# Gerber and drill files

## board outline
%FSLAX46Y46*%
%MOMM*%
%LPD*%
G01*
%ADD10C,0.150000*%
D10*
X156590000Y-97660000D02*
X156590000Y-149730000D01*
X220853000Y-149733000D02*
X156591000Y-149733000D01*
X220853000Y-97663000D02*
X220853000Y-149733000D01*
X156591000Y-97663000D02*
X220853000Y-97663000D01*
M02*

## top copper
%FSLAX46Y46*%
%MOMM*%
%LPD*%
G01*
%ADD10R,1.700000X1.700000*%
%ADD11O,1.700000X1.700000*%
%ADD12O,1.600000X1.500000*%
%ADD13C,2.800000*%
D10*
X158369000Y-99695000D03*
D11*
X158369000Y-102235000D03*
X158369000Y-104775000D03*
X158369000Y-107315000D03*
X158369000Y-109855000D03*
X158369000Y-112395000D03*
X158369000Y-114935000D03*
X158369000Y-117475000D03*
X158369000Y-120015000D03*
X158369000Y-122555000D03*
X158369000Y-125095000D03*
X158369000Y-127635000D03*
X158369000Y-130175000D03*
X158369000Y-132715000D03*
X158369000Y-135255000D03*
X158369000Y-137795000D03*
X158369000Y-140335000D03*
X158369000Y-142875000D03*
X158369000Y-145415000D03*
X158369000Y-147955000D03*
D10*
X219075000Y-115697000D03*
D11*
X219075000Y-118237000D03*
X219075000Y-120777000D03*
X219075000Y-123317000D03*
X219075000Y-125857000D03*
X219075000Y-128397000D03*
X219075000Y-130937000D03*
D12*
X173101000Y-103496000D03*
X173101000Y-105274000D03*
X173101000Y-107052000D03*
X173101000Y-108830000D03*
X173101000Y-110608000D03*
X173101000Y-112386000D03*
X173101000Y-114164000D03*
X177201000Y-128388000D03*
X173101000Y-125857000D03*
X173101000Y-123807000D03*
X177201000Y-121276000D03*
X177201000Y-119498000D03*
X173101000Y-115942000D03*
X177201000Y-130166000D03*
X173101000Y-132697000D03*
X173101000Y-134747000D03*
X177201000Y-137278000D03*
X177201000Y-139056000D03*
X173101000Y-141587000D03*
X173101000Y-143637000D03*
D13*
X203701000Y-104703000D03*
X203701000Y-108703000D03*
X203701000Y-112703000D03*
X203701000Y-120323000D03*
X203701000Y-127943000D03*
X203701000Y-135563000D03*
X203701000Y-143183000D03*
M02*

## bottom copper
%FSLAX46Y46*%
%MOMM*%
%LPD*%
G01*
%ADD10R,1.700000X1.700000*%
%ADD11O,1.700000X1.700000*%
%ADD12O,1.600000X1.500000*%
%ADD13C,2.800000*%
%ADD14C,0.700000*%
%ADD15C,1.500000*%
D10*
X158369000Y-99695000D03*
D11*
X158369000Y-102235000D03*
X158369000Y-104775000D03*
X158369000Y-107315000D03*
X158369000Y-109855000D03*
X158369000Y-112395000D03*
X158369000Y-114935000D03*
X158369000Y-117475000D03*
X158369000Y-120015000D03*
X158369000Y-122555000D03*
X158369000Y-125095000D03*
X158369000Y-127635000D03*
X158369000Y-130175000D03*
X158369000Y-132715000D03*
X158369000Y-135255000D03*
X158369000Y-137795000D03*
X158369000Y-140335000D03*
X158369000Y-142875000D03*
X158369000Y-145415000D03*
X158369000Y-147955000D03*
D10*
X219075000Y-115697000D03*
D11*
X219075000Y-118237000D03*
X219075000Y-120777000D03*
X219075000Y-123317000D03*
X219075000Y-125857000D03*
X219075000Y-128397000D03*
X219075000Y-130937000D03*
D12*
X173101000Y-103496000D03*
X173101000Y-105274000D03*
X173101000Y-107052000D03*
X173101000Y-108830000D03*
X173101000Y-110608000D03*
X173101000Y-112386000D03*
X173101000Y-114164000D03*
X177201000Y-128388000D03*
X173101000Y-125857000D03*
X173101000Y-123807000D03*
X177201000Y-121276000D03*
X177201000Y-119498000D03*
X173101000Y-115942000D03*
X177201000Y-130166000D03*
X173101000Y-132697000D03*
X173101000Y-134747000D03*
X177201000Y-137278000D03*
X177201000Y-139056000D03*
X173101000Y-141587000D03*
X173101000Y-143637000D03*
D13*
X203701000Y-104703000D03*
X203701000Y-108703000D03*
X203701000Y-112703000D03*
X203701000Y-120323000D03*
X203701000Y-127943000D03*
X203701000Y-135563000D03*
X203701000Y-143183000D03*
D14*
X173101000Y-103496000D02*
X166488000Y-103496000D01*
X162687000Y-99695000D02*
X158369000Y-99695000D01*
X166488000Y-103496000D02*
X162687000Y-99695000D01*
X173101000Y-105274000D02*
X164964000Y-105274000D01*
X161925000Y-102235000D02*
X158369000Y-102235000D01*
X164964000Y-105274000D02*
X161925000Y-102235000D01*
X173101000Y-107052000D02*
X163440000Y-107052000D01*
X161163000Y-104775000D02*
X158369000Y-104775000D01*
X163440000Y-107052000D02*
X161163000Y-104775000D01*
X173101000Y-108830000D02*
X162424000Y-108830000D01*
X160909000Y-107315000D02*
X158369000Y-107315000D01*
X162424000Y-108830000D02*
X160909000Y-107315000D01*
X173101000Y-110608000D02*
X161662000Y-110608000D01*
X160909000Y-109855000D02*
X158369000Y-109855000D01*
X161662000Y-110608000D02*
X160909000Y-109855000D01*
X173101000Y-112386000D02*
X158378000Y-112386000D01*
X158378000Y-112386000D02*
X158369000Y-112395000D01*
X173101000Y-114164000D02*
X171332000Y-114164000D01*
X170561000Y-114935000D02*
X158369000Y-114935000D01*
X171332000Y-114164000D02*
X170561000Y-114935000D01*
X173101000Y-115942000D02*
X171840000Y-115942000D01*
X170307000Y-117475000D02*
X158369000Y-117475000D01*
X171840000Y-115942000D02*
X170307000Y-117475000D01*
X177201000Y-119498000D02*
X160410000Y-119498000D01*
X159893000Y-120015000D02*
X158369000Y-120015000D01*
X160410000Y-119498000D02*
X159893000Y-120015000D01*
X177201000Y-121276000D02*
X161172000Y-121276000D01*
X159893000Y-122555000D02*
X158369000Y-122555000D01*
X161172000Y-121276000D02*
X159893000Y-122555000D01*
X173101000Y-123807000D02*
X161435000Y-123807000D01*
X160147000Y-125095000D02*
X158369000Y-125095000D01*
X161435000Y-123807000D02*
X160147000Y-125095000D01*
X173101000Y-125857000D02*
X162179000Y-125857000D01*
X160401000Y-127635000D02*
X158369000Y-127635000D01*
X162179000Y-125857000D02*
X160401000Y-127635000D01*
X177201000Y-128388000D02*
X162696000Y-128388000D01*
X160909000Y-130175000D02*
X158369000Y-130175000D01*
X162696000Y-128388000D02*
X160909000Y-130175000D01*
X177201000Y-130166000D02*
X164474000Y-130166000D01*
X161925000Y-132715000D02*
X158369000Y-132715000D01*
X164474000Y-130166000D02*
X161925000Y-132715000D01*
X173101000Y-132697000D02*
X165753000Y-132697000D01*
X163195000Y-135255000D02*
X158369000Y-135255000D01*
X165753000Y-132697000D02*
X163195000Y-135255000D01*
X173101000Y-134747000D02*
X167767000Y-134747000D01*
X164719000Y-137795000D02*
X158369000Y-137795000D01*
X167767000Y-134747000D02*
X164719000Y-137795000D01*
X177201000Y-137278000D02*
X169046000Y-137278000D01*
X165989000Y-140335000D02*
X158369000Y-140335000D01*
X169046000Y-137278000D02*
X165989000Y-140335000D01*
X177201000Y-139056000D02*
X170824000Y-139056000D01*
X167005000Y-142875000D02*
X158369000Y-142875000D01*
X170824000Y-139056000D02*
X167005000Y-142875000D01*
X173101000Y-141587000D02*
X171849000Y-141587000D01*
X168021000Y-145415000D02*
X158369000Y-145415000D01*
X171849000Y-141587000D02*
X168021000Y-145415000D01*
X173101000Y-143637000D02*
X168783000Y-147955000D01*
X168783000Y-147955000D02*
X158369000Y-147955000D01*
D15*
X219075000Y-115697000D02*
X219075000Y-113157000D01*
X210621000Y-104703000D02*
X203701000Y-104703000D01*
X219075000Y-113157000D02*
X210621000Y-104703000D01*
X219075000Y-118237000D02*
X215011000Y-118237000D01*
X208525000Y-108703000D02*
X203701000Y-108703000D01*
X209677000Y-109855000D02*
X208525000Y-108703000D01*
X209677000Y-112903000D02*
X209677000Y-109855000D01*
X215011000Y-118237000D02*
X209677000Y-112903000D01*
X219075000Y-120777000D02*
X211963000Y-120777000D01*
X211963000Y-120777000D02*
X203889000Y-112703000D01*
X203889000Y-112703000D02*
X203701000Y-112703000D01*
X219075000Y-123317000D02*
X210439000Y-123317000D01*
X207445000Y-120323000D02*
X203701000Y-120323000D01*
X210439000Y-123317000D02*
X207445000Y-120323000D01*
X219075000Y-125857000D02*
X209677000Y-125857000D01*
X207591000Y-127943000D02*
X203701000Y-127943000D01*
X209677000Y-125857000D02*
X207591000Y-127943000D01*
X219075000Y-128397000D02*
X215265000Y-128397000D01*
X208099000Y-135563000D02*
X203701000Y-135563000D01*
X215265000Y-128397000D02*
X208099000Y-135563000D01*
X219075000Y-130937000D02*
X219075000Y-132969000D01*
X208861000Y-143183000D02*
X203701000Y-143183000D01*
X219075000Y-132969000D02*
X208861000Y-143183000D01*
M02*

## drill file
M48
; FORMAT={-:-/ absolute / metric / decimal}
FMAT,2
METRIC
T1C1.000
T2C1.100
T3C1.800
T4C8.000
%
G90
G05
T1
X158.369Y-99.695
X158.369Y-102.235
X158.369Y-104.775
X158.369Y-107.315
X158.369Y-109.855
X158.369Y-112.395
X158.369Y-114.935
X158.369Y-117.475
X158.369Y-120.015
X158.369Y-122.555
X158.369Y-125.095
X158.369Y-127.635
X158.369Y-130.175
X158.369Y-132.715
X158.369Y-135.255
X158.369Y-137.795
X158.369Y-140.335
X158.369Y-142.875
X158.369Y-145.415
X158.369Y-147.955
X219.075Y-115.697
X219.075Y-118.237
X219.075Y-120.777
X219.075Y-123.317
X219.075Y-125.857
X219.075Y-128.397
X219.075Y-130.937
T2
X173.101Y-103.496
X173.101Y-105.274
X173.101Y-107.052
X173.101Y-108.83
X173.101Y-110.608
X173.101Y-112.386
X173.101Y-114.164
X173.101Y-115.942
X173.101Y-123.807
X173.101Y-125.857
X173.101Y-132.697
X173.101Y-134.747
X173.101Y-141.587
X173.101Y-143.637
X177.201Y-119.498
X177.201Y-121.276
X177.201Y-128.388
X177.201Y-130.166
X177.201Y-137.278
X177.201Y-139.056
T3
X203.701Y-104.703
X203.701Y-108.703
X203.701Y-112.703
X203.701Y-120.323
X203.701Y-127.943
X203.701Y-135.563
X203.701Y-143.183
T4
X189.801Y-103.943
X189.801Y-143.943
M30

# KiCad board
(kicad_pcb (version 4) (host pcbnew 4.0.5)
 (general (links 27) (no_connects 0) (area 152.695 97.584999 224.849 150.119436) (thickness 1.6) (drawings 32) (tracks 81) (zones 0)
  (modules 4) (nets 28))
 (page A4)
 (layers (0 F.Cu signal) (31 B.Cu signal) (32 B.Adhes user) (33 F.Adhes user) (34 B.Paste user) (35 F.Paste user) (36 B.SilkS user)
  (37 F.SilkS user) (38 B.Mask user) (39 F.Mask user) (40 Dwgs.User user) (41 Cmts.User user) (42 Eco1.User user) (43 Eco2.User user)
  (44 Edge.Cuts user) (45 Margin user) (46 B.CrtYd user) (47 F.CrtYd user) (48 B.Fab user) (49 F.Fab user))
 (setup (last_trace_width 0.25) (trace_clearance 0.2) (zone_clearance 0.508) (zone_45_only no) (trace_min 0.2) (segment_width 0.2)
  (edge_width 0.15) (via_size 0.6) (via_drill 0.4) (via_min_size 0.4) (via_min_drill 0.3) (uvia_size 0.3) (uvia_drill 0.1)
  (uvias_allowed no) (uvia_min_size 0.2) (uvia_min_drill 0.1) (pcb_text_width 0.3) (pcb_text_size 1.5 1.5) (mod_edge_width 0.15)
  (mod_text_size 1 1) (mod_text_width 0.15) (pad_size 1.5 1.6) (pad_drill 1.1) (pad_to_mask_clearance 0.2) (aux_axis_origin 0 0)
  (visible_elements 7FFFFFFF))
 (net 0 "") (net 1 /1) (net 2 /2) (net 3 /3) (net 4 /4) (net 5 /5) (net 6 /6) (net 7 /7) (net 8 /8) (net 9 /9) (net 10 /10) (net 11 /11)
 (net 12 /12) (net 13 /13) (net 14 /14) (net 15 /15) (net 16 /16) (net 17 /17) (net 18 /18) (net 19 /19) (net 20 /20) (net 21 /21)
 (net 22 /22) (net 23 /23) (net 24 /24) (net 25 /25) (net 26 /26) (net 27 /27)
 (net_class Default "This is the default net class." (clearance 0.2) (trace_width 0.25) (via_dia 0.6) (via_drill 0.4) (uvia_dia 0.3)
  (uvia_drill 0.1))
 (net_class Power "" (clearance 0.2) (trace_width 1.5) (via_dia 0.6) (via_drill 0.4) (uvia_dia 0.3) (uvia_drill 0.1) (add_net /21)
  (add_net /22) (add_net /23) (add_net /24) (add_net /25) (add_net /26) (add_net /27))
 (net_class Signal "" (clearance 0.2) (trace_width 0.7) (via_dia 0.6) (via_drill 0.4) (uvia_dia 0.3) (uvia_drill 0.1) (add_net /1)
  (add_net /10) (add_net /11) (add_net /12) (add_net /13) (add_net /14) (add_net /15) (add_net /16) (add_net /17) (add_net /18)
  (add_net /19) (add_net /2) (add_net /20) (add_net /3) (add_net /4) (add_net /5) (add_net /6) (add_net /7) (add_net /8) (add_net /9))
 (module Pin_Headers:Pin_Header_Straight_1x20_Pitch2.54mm (layer F.Cu) (at 158.369 99.695)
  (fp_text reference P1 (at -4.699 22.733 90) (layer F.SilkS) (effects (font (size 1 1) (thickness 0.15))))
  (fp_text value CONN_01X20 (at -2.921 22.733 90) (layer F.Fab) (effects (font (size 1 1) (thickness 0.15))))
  (pad 1 thru_hole rect (at 0 0) (size 1.7 1.7) (drill 1) (layers *.Cu *.Mask) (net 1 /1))
  (pad 2 thru_hole oval (at 0 2.54) (size 1.7 1.7) (drill 1) (layers *.Cu *.Mask) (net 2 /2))
  (pad 3 thru_hole oval (at 0 5.08) (size 1.7 1.7) (drill 1) (layers *.Cu *.Mask) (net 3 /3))
  (pad 4 thru_hole oval (at 0 7.62) (size 1.7 1.7) (drill 1) (layers *.Cu *.Mask) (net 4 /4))
  (pad 5 thru_hole oval (at 0 10.16) (size 1.7 1.7) (drill 1) (layers *.Cu *.Mask) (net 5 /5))
  (pad 6 thru_hole oval (at 0 12.7) (size 1.7 1.7) (drill 1) (layers *.Cu *.Mask) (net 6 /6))
  (pad 7 thru_hole oval (at 0 15.24) (size 1.7 1.7) (drill 1) (layers *.Cu *.Mask) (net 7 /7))
  (pad 8 thru_hole oval (at 0 17.78) (size 1.7 1.7) (drill 1) (layers *.Cu *.Mask) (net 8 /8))
  (pad 9 thru_hole oval (at 0 20.32) (size 1.7 1.7) (drill 1) (layers *.Cu *.Mask) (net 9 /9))
  (pad 10 thru_hole oval (at 0 22.86) (size 1.7 1.7) (drill 1) (layers *.Cu *.Mask) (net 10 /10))
  (pad 11 thru_hole oval (at 0 25.4) (size 1.7 1.7) (drill 1) (layers *.Cu *.Mask) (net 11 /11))
  (pad 12 thru_hole oval (at 0 27.94) (size 1.7 1.7) (drill 1) (layers *.Cu *.Mask) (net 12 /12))
  (pad 13 thru_hole oval (at 0 30.48) (size 1.7 1.7) (drill 1) (layers *.Cu *.Mask) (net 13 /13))
  (pad 14 thru_hole oval (at 0 33.02) (size 1.7 1.7) (drill 1) (layers *.Cu *.Mask) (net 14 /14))
  (pad 15 thru_hole oval (at 0 35.56) (size 1.7 1.7) (drill 1) (layers *.Cu *.Mask) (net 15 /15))
  (pad 16 thru_hole oval (at 0 38.1) (size 1.7 1.7) (drill 1) (layers *.Cu *.Mask) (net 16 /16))
  (pad 17 thru_hole oval (at 0 40.64) (size 1.7 1.7) (drill 1) (layers *.Cu *.Mask) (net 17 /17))
  (pad 18 thru_hole oval (at 0 43.18) (size 1.7 1.7) (drill 1) (layers *.Cu *.Mask) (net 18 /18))
  (pad 19 thru_hole oval (at 0 45.72) (size 1.7 1.7) (drill 1) (layers *.Cu *.Mask) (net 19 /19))
  (pad 20 thru_hole oval (at 0 48.26) (size 1.7 1.7) (drill 1) (layers *.Cu *.Mask) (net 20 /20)))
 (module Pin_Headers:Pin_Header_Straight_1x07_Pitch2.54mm (layer F.Cu) (at 219.075 115.697)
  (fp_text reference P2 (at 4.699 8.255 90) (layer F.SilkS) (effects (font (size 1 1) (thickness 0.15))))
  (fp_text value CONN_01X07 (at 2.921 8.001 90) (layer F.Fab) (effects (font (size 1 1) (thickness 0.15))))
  (pad 1 thru_hole rect (at 0 0) (size 1.7 1.7) (drill 1) (layers *.Cu *.Mask) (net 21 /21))
  (pad 2 thru_hole oval (at 0 2.54) (size 1.7 1.7) (drill 1) (layers *.Cu *.Mask) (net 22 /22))
  (pad 3 thru_hole oval (at 0 5.08) (size 1.7 1.7) (drill 1) (layers *.Cu *.Mask) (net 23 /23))
  (pad 4 thru_hole oval (at 0 7.62) (size 1.7 1.7) (drill 1) (layers *.Cu *.Mask) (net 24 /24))
  (pad 5 thru_hole oval (at 0 10.16) (size 1.7 1.7) (drill 1) (layers *.Cu *.Mask) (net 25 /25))
  (pad 6 thru_hole oval (at 0 12.7) (size 1.7 1.7) (drill 1) (layers *.Cu *.Mask) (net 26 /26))
  (pad 7 thru_hole oval (at 0 15.24) (size 1.7 1.7) (drill 1) (layers *.Cu *.Mask) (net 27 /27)))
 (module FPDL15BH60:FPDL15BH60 (layer F.Cu) (at 173.101 143.637 90)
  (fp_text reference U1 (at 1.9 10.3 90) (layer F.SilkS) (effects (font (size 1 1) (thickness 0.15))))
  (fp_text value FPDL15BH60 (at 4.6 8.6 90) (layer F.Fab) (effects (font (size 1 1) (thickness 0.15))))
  (pad 1 thru_hole oval (at 40.141 0 90) (size 1.5 1.6) (drill 1.1) (layers *.Cu *.Mask) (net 1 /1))
  (pad 2 thru_hole oval (at 38.363 0 90) (size 1.5 1.6) (drill 1.1) (layers *.Cu *.Mask) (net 2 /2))
  (pad 3 thru_hole oval (at 36.585 0 90) (size 1.5 1.6) (drill 1.1) (layers *.Cu *.Mask) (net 3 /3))
  (pad 4 thru_hole oval (at 34.807 0 90) (size 1.5 1.6) (drill 1.1) (layers *.Cu) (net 4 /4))
  (pad 5 thru_hole oval (at 33.029 0 90) (size 1.5 1.6) (drill 1.1) (layers *.Cu *.Mask) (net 5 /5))
  (pad 6 thru_hole oval (at 31.251 0 90) (size 1.5 1.6) (drill 1.1) (layers *.Cu *.Mask) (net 6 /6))
  (pad 7 thru_hole oval (at 29.473 0 90) (size 1.5 1.6) (drill 1.1) (layers *.Cu *.Mask) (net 7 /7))
  (pad 13 thru_hole oval (at 15.249 4.1 90) (size 1.5 1.6) (drill 1.1) (layers *.Cu *.Mask) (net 13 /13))
  (pad 12 thru_hole oval (at 17.78 0 90) (size 1.5 1.6) (drill 1.1) (layers *.Cu *.Mask) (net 12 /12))
  (pad 11 thru_hole oval (at 19.83 0 90) (size 1.5 1.6) (drill 1.1) (layers *.Cu *.Mask) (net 11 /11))
  (pad 10 thru_hole oval (at 22.361 4.1 90) (size 1.5 1.6) (drill 1.1) (layers *.Cu *.Mask) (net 10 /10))
  (pad 9 thru_hole oval (at 24.139 4.1 90) (size 1.5 1.6) (drill 1.1) (layers *.Cu *.Mask) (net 9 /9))
  (pad 8 thru_hole oval (at 27.695 0 90) (size 1.5 1.6) (drill 1.1) (layers *.Cu *.Mask) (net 8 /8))
  (pad 14 thru_hole oval (at 13.471 4.1 90) (size 1.5 1.6) (drill 1.1) (layers *.Cu *.Mask) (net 14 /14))
  (pad 15 thru_hole oval (at 10.94 0 90) (size 1.5 1.6) (drill 1.1) (layers *.Cu *.Mask) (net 15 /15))
  (pad 16 thru_hole oval (at 8.89 0 90) (size 1.5 1.6) (drill 1.1) (layers *.Cu *.Mask) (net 16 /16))
  (pad 17 thru_hole oval (at 6.359 4.1 90) (size 1.5 1.6) (drill 1.1) (layers *.Cu *.Mask) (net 17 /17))
  (pad 18 thru_hole oval (at 4.581 4.1 90) (size 1.5 1.6) (drill 1.1) (layers *.Cu *.Mask) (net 18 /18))
  (pad 19 thru_hole oval (at 2.05 0 90) (size 1.5 1.6) (drill 1.1) (layers *.Cu *.Mask) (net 19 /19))
  (pad 20 thru_hole oval (at 0 0 90) (size 1.5 1.6) (drill 1.1) (layers *.Cu *.Mask) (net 20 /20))
  (pad 21 thru_hole circle (at 38.934 30.6 90) (size 2.8 2.8) (drill 1.8) (layers *.Cu *.Mask) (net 21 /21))
  (pad 22 thru_hole circle (at 34.934 30.6 90) (size 2.8 2.8) (drill 1.8) (layers *.Cu *.Mask) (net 22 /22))
  (pad 23 thru_hole circle (at 30.934 30.6 90) (size 2.8 2.8) (drill 1.8) (layers *.Cu *.Mask) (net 23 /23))
  (pad 24 thru_hole circle (at 23.314 30.6 90) (size 2.8 2.8) (drill 1.8) (layers *.Cu *.Mask) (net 24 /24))
  (pad 25 thru_hole circle (at 15.694 30.6 90) (size 2.8 2.8) (drill 1.8) (layers *.Cu *.Mask) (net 25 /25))
  (pad 26 thru_hole circle (at 8.074 30.6 90) (size 2.8 2.8) (drill 1.8) (layers *.Cu *.Mask) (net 26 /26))
  (pad 27 thru_hole circle (at 0.454 30.6 90) (size 2.8 2.8) (drill 1.8) (layers *.Cu *.Mask) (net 27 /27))
  (pad "" np_thru_hole circle (at -0.306 16.7 90) (size 8 8) (drill 8) (layers *.Cu))
  (pad "" np_thru_hole circle (at 39.694 16.7 90) (size 8 8) (drill 8) (layers *.Cu)))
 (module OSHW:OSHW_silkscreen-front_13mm (layer F.Cu) (at 212.852 142.494)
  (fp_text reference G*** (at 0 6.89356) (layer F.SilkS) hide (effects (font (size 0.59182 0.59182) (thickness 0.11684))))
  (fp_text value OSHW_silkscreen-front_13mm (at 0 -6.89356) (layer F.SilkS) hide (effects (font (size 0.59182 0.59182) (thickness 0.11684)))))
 (gr_line (start 156.59 97.66) (end 156.59 149.73) (angle 90) (layer Edge.Cuts) (width 0.15))
 (gr_line (start 220.853 149.733) (end 156.591 149.733) (angle 90) (layer Edge.Cuts) (width 0.15))
 (gr_line (start 220.853 97.663) (end 220.853 149.733) (angle 90) (layer Edge.Cuts) (width 0.15))
 (gr_line (start 156.591 97.663) (end 220.853 97.663) (angle 90) (layer Edge.Cuts) (width 0.15))
 (segment (start 173.101 103.496) (end 166.488 103.496) (width 0.7) (layer B.Cu) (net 1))
 (segment (start 162.687 99.695) (end 158.369 99.695) (width 0.7) (layer B.Cu) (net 1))
 (segment (start 166.488 103.496) (end 162.687 99.695) (width 0.7) (layer B.Cu) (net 1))
 (segment (start 173.101 105.274) (end 164.964 105.274) (width 0.7) (layer B.Cu) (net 2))
 (segment (start 161.925 102.235) (end 158.369 102.235) (width 0.7) (layer B.Cu) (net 2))
 (segment (start 164.964 105.274) (end 161.925 102.235) (width 0.7) (layer B.Cu) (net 2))
 (segment (start 173.101 107.052) (end 163.44 107.052) (width 0.7) (layer B.Cu) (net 3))
 (segment (start 161.163 104.775) (end 158.369 104.775) (width 0.7) (layer B.Cu) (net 3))
 (segment (start 163.44 107.052) (end 161.163 104.775) (width 0.7) (layer B.Cu) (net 3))
 (segment (start 173.101 108.83) (end 162.424 108.83) (width 0.7) (layer B.Cu) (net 4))
 (segment (start 160.909 107.315) (end 158.369 107.315) (width 0.7) (layer B.Cu) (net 4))
 (segment (start 162.424 108.83) (end 160.909 107.315) (width 0.7) (layer B.Cu) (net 4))
 (segment (start 173.101 110.608) (end 161.662 110.608) (width 0.7) (layer B.Cu) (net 5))
 (segment (start 160.909 109.855) (end 158.369 109.855) (width 0.7) (layer B.Cu) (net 5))
 (segment (start 161.662 110.608) (end 160.909 109.855) (width 0.7) (layer B.Cu) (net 5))
 (segment (start 173.101 112.386) (end 158.378 112.386) (width 0.7) (layer B.Cu) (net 6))
 (segment (start 158.378 112.386) (end 158.369 112.395) (width 0.7) (layer B.Cu) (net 6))
 (segment (start 173.101 114.164) (end 171.332 114.164) (width 0.7) (layer B.Cu) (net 7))
 (segment (start 170.561 114.935) (end 158.369 114.935) (width 0.7) (layer B.Cu) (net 7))
 (segment (start 171.332 114.164) (end 170.561 114.935) (width 0.7) (layer B.Cu) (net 7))
 (segment (start 173.101 115.942) (end 171.84 115.942) (width 0.7) (layer B.Cu) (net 8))
 (segment (start 170.307 117.475) (end 158.369 117.475) (width 0.7) (layer B.Cu) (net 8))
 (segment (start 171.84 115.942) (end 170.307 117.475) (width 0.7) (layer B.Cu) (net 8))
 (segment (start 177.201 119.498) (end 160.41 119.498) (width 0.7) (layer B.Cu) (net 9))
 (segment (start 159.893 120.015) (end 158.369 120.015) (width 0.7) (layer B.Cu) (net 9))
 (segment (start 160.41 119.498) (end 159.893 120.015) (width 0.7) (layer B.Cu) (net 9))
 (segment (start 177.201 121.276) (end 161.172 121.276) (width 0.7) (layer B.Cu) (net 10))
 (segment (start 159.893 122.555) (end 158.369 122.555) (width 0.7) (layer B.Cu) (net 10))
 (segment (start 161.172 121.276) (end 159.893 122.555) (width 0.7) (layer B.Cu) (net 10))
 (segment (start 173.101 123.807) (end 161.435 123.807) (width 0.7) (layer B.Cu) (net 11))
 (segment (start 160.147 125.095) (end 158.369 125.095) (width 0.7) (layer B.Cu) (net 11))
 (segment (start 161.435 123.807) (end 160.147 125.095) (width 0.7) (layer B.Cu) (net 11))
 (segment (start 173.101 125.857) (end 162.179 125.857) (width 0.7) (layer B.Cu) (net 12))
 (segment (start 160.401 127.635) (end 158.369 127.635) (width 0.7) (layer B.Cu) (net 12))
 (segment (start 162.179 125.857) (end 160.401 127.635) (width 0.7) (layer B.Cu) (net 12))
 (segment (start 177.201 128.388) (end 162.696 128.388) (width 0.7) (layer B.Cu) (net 13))
 (segment (start 160.909 130.175) (end 158.369 130.175) (width 0.7) (layer B.Cu) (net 13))
 (segment (start 162.696 128.388) (end 160.909 130.175) (width 0.7) (layer B.Cu) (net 13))
 (segment (start 177.201 130.166) (end 164.474 130.166) (width 0.7) (layer B.Cu) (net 14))
 (segment (start 161.925 132.715) (end 158.369 132.715) (width 0.7) (layer B.Cu) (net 14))
 (segment (start 164.474 130.166) (end 161.925 132.715) (width 0.7) (layer B.Cu) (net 14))
 (segment (start 173.101 132.697) (end 165.753 132.697) (width 0.7) (layer B.Cu) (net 15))
 (segment (start 163.195 135.255) (end 158.369 135.255) (width 0.7) (layer B.Cu) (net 15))
 (segment (start 165.753 132.697) (end 163.195 135.255) (width 0.7) (layer B.Cu) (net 15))
 (segment (start 173.101 134.747) (end 167.767 134.747) (width 0.7) (layer B.Cu) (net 16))
 (segment (start 164.719 137.795) (end 158.369 137.795) (width 0.7) (layer B.Cu) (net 16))
 (segment (start 167.767 134.747) (end 164.719 137.795) (width 0.7) (layer B.Cu) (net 16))
 (segment (start 177.201 137.278) (end 169.046 137.278) (width 0.7) (layer B.Cu) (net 17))
 (segment (start 165.989 140.335) (end 158.369 140.335) (width 0.7) (layer B.Cu) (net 17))
 (segment (start 169.046 137.278) (end 165.989 140.335) (width 0.7) (layer B.Cu) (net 17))
 (segment (start 177.201 139.056) (end 170.824 139.056) (width 0.7) (layer B.Cu) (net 18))
 (segment (start 167.005 142.875) (end 158.369 142.875) (width 0.7) (layer B.Cu) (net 18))
 (segment (start 170.824 139.056) (end 167.005 142.875) (width 0.7) (layer B.Cu) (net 18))
 (segment (start 173.101 141.587) (end 171.849 141.587) (width 0.7) (layer B.Cu) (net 19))
 (segment (start 168.021 145.415) (end 158.369 145.415) (width 0.7) (layer B.Cu) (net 19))
 (segment (start 171.849 141.587) (end 168.021 145.415) (width 0.7) (layer B.Cu) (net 19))
 (segment (start 173.101 143.637) (end 168.783 147.955) (width 0.7) (layer B.Cu) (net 20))
 (segment (start 168.783 147.955) (end 158.369 147.955) (width 0.7) (layer B.Cu) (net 20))
 (segment (start 219.075 115.697) (end 219.075 113.157) (width 1.5) (layer B.Cu) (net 21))
 (segment (start 210.621 104.703) (end 203.701 104.703) (width 1.5) (layer B.Cu) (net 21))
 (segment (start 219.075 113.157) (end 210.621 104.703) (width 1.5) (layer B.Cu) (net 21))
 (segment (start 219.075 118.237) (end 215.011 118.237) (width 1.5) (layer B.Cu) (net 22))
 (segment (start 208.525 108.703) (end 203.701 108.703) (width 1.5) (layer B.Cu) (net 22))
 (segment (start 209.677 109.855) (end 208.525 108.703) (width 1.5) (layer B.Cu) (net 22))
 (segment (start 209.677 112.903) (end 209.677 109.855) (width 1.5) (layer B.Cu) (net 22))
 (segment (start 215.011 118.237) (end 209.677 112.903) (width 1.5) (layer B.Cu) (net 22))
 (segment (start 219.075 120.777) (end 211.963 120.777) (width 1.5) (layer B.Cu) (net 23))
 (segment (start 211.963 120.777) (end 203.889 112.703) (width 1.5) (layer B.Cu) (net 23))
 (segment (start 203.889 112.703) (end 203.701 112.703) (width 1.5) (layer B.Cu) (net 23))
 (segment (start 219.075 123.317) (end 210.439 123.317) (width 1.5) (layer B.Cu) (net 24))
 (segment (start 207.445 120.323) (end 203.701 120.323) (width 1.5) (layer B.Cu) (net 24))
 (segment (start 210.439 123.317) (end 207.445 120.323) (width 1.5) (layer B.Cu) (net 24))
 (segment (start 219.075 125.857) (end 209.677 125.857) (width 1.5) (layer B.Cu) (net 25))
 (segment (start 207.591 127.943) (end 203.701 127.943) (width 1.5) (layer B.Cu) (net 25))
 (segment (start 209.677 125.857) (end 207.591 127.943) (width 1.5) (layer B.Cu) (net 25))
 (segment (start 219.075 128.397) (end 215.265 128.397) (width 1.5) (layer B.Cu) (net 26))
 (segment (start 208.099 135.563) (end 203.701 135.563) (width 1.5) (layer B.Cu) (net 26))
 (segment (start 215.265 128.397) (end 208.099 135.563) (width 1.5) (layer B.Cu) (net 26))
 (segment (start 219.075 130.937) (end 219.075 132.969) (width 1.5) (layer B.Cu) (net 27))
 (segment (start 208.861 143.183) (end 203.701 143.183) (width 1.5) (layer B.Cu) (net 27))
 (segment (start 219.075 132.969) (end 208.861 143.183) (width 1.5) (layer B.Cu) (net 27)))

